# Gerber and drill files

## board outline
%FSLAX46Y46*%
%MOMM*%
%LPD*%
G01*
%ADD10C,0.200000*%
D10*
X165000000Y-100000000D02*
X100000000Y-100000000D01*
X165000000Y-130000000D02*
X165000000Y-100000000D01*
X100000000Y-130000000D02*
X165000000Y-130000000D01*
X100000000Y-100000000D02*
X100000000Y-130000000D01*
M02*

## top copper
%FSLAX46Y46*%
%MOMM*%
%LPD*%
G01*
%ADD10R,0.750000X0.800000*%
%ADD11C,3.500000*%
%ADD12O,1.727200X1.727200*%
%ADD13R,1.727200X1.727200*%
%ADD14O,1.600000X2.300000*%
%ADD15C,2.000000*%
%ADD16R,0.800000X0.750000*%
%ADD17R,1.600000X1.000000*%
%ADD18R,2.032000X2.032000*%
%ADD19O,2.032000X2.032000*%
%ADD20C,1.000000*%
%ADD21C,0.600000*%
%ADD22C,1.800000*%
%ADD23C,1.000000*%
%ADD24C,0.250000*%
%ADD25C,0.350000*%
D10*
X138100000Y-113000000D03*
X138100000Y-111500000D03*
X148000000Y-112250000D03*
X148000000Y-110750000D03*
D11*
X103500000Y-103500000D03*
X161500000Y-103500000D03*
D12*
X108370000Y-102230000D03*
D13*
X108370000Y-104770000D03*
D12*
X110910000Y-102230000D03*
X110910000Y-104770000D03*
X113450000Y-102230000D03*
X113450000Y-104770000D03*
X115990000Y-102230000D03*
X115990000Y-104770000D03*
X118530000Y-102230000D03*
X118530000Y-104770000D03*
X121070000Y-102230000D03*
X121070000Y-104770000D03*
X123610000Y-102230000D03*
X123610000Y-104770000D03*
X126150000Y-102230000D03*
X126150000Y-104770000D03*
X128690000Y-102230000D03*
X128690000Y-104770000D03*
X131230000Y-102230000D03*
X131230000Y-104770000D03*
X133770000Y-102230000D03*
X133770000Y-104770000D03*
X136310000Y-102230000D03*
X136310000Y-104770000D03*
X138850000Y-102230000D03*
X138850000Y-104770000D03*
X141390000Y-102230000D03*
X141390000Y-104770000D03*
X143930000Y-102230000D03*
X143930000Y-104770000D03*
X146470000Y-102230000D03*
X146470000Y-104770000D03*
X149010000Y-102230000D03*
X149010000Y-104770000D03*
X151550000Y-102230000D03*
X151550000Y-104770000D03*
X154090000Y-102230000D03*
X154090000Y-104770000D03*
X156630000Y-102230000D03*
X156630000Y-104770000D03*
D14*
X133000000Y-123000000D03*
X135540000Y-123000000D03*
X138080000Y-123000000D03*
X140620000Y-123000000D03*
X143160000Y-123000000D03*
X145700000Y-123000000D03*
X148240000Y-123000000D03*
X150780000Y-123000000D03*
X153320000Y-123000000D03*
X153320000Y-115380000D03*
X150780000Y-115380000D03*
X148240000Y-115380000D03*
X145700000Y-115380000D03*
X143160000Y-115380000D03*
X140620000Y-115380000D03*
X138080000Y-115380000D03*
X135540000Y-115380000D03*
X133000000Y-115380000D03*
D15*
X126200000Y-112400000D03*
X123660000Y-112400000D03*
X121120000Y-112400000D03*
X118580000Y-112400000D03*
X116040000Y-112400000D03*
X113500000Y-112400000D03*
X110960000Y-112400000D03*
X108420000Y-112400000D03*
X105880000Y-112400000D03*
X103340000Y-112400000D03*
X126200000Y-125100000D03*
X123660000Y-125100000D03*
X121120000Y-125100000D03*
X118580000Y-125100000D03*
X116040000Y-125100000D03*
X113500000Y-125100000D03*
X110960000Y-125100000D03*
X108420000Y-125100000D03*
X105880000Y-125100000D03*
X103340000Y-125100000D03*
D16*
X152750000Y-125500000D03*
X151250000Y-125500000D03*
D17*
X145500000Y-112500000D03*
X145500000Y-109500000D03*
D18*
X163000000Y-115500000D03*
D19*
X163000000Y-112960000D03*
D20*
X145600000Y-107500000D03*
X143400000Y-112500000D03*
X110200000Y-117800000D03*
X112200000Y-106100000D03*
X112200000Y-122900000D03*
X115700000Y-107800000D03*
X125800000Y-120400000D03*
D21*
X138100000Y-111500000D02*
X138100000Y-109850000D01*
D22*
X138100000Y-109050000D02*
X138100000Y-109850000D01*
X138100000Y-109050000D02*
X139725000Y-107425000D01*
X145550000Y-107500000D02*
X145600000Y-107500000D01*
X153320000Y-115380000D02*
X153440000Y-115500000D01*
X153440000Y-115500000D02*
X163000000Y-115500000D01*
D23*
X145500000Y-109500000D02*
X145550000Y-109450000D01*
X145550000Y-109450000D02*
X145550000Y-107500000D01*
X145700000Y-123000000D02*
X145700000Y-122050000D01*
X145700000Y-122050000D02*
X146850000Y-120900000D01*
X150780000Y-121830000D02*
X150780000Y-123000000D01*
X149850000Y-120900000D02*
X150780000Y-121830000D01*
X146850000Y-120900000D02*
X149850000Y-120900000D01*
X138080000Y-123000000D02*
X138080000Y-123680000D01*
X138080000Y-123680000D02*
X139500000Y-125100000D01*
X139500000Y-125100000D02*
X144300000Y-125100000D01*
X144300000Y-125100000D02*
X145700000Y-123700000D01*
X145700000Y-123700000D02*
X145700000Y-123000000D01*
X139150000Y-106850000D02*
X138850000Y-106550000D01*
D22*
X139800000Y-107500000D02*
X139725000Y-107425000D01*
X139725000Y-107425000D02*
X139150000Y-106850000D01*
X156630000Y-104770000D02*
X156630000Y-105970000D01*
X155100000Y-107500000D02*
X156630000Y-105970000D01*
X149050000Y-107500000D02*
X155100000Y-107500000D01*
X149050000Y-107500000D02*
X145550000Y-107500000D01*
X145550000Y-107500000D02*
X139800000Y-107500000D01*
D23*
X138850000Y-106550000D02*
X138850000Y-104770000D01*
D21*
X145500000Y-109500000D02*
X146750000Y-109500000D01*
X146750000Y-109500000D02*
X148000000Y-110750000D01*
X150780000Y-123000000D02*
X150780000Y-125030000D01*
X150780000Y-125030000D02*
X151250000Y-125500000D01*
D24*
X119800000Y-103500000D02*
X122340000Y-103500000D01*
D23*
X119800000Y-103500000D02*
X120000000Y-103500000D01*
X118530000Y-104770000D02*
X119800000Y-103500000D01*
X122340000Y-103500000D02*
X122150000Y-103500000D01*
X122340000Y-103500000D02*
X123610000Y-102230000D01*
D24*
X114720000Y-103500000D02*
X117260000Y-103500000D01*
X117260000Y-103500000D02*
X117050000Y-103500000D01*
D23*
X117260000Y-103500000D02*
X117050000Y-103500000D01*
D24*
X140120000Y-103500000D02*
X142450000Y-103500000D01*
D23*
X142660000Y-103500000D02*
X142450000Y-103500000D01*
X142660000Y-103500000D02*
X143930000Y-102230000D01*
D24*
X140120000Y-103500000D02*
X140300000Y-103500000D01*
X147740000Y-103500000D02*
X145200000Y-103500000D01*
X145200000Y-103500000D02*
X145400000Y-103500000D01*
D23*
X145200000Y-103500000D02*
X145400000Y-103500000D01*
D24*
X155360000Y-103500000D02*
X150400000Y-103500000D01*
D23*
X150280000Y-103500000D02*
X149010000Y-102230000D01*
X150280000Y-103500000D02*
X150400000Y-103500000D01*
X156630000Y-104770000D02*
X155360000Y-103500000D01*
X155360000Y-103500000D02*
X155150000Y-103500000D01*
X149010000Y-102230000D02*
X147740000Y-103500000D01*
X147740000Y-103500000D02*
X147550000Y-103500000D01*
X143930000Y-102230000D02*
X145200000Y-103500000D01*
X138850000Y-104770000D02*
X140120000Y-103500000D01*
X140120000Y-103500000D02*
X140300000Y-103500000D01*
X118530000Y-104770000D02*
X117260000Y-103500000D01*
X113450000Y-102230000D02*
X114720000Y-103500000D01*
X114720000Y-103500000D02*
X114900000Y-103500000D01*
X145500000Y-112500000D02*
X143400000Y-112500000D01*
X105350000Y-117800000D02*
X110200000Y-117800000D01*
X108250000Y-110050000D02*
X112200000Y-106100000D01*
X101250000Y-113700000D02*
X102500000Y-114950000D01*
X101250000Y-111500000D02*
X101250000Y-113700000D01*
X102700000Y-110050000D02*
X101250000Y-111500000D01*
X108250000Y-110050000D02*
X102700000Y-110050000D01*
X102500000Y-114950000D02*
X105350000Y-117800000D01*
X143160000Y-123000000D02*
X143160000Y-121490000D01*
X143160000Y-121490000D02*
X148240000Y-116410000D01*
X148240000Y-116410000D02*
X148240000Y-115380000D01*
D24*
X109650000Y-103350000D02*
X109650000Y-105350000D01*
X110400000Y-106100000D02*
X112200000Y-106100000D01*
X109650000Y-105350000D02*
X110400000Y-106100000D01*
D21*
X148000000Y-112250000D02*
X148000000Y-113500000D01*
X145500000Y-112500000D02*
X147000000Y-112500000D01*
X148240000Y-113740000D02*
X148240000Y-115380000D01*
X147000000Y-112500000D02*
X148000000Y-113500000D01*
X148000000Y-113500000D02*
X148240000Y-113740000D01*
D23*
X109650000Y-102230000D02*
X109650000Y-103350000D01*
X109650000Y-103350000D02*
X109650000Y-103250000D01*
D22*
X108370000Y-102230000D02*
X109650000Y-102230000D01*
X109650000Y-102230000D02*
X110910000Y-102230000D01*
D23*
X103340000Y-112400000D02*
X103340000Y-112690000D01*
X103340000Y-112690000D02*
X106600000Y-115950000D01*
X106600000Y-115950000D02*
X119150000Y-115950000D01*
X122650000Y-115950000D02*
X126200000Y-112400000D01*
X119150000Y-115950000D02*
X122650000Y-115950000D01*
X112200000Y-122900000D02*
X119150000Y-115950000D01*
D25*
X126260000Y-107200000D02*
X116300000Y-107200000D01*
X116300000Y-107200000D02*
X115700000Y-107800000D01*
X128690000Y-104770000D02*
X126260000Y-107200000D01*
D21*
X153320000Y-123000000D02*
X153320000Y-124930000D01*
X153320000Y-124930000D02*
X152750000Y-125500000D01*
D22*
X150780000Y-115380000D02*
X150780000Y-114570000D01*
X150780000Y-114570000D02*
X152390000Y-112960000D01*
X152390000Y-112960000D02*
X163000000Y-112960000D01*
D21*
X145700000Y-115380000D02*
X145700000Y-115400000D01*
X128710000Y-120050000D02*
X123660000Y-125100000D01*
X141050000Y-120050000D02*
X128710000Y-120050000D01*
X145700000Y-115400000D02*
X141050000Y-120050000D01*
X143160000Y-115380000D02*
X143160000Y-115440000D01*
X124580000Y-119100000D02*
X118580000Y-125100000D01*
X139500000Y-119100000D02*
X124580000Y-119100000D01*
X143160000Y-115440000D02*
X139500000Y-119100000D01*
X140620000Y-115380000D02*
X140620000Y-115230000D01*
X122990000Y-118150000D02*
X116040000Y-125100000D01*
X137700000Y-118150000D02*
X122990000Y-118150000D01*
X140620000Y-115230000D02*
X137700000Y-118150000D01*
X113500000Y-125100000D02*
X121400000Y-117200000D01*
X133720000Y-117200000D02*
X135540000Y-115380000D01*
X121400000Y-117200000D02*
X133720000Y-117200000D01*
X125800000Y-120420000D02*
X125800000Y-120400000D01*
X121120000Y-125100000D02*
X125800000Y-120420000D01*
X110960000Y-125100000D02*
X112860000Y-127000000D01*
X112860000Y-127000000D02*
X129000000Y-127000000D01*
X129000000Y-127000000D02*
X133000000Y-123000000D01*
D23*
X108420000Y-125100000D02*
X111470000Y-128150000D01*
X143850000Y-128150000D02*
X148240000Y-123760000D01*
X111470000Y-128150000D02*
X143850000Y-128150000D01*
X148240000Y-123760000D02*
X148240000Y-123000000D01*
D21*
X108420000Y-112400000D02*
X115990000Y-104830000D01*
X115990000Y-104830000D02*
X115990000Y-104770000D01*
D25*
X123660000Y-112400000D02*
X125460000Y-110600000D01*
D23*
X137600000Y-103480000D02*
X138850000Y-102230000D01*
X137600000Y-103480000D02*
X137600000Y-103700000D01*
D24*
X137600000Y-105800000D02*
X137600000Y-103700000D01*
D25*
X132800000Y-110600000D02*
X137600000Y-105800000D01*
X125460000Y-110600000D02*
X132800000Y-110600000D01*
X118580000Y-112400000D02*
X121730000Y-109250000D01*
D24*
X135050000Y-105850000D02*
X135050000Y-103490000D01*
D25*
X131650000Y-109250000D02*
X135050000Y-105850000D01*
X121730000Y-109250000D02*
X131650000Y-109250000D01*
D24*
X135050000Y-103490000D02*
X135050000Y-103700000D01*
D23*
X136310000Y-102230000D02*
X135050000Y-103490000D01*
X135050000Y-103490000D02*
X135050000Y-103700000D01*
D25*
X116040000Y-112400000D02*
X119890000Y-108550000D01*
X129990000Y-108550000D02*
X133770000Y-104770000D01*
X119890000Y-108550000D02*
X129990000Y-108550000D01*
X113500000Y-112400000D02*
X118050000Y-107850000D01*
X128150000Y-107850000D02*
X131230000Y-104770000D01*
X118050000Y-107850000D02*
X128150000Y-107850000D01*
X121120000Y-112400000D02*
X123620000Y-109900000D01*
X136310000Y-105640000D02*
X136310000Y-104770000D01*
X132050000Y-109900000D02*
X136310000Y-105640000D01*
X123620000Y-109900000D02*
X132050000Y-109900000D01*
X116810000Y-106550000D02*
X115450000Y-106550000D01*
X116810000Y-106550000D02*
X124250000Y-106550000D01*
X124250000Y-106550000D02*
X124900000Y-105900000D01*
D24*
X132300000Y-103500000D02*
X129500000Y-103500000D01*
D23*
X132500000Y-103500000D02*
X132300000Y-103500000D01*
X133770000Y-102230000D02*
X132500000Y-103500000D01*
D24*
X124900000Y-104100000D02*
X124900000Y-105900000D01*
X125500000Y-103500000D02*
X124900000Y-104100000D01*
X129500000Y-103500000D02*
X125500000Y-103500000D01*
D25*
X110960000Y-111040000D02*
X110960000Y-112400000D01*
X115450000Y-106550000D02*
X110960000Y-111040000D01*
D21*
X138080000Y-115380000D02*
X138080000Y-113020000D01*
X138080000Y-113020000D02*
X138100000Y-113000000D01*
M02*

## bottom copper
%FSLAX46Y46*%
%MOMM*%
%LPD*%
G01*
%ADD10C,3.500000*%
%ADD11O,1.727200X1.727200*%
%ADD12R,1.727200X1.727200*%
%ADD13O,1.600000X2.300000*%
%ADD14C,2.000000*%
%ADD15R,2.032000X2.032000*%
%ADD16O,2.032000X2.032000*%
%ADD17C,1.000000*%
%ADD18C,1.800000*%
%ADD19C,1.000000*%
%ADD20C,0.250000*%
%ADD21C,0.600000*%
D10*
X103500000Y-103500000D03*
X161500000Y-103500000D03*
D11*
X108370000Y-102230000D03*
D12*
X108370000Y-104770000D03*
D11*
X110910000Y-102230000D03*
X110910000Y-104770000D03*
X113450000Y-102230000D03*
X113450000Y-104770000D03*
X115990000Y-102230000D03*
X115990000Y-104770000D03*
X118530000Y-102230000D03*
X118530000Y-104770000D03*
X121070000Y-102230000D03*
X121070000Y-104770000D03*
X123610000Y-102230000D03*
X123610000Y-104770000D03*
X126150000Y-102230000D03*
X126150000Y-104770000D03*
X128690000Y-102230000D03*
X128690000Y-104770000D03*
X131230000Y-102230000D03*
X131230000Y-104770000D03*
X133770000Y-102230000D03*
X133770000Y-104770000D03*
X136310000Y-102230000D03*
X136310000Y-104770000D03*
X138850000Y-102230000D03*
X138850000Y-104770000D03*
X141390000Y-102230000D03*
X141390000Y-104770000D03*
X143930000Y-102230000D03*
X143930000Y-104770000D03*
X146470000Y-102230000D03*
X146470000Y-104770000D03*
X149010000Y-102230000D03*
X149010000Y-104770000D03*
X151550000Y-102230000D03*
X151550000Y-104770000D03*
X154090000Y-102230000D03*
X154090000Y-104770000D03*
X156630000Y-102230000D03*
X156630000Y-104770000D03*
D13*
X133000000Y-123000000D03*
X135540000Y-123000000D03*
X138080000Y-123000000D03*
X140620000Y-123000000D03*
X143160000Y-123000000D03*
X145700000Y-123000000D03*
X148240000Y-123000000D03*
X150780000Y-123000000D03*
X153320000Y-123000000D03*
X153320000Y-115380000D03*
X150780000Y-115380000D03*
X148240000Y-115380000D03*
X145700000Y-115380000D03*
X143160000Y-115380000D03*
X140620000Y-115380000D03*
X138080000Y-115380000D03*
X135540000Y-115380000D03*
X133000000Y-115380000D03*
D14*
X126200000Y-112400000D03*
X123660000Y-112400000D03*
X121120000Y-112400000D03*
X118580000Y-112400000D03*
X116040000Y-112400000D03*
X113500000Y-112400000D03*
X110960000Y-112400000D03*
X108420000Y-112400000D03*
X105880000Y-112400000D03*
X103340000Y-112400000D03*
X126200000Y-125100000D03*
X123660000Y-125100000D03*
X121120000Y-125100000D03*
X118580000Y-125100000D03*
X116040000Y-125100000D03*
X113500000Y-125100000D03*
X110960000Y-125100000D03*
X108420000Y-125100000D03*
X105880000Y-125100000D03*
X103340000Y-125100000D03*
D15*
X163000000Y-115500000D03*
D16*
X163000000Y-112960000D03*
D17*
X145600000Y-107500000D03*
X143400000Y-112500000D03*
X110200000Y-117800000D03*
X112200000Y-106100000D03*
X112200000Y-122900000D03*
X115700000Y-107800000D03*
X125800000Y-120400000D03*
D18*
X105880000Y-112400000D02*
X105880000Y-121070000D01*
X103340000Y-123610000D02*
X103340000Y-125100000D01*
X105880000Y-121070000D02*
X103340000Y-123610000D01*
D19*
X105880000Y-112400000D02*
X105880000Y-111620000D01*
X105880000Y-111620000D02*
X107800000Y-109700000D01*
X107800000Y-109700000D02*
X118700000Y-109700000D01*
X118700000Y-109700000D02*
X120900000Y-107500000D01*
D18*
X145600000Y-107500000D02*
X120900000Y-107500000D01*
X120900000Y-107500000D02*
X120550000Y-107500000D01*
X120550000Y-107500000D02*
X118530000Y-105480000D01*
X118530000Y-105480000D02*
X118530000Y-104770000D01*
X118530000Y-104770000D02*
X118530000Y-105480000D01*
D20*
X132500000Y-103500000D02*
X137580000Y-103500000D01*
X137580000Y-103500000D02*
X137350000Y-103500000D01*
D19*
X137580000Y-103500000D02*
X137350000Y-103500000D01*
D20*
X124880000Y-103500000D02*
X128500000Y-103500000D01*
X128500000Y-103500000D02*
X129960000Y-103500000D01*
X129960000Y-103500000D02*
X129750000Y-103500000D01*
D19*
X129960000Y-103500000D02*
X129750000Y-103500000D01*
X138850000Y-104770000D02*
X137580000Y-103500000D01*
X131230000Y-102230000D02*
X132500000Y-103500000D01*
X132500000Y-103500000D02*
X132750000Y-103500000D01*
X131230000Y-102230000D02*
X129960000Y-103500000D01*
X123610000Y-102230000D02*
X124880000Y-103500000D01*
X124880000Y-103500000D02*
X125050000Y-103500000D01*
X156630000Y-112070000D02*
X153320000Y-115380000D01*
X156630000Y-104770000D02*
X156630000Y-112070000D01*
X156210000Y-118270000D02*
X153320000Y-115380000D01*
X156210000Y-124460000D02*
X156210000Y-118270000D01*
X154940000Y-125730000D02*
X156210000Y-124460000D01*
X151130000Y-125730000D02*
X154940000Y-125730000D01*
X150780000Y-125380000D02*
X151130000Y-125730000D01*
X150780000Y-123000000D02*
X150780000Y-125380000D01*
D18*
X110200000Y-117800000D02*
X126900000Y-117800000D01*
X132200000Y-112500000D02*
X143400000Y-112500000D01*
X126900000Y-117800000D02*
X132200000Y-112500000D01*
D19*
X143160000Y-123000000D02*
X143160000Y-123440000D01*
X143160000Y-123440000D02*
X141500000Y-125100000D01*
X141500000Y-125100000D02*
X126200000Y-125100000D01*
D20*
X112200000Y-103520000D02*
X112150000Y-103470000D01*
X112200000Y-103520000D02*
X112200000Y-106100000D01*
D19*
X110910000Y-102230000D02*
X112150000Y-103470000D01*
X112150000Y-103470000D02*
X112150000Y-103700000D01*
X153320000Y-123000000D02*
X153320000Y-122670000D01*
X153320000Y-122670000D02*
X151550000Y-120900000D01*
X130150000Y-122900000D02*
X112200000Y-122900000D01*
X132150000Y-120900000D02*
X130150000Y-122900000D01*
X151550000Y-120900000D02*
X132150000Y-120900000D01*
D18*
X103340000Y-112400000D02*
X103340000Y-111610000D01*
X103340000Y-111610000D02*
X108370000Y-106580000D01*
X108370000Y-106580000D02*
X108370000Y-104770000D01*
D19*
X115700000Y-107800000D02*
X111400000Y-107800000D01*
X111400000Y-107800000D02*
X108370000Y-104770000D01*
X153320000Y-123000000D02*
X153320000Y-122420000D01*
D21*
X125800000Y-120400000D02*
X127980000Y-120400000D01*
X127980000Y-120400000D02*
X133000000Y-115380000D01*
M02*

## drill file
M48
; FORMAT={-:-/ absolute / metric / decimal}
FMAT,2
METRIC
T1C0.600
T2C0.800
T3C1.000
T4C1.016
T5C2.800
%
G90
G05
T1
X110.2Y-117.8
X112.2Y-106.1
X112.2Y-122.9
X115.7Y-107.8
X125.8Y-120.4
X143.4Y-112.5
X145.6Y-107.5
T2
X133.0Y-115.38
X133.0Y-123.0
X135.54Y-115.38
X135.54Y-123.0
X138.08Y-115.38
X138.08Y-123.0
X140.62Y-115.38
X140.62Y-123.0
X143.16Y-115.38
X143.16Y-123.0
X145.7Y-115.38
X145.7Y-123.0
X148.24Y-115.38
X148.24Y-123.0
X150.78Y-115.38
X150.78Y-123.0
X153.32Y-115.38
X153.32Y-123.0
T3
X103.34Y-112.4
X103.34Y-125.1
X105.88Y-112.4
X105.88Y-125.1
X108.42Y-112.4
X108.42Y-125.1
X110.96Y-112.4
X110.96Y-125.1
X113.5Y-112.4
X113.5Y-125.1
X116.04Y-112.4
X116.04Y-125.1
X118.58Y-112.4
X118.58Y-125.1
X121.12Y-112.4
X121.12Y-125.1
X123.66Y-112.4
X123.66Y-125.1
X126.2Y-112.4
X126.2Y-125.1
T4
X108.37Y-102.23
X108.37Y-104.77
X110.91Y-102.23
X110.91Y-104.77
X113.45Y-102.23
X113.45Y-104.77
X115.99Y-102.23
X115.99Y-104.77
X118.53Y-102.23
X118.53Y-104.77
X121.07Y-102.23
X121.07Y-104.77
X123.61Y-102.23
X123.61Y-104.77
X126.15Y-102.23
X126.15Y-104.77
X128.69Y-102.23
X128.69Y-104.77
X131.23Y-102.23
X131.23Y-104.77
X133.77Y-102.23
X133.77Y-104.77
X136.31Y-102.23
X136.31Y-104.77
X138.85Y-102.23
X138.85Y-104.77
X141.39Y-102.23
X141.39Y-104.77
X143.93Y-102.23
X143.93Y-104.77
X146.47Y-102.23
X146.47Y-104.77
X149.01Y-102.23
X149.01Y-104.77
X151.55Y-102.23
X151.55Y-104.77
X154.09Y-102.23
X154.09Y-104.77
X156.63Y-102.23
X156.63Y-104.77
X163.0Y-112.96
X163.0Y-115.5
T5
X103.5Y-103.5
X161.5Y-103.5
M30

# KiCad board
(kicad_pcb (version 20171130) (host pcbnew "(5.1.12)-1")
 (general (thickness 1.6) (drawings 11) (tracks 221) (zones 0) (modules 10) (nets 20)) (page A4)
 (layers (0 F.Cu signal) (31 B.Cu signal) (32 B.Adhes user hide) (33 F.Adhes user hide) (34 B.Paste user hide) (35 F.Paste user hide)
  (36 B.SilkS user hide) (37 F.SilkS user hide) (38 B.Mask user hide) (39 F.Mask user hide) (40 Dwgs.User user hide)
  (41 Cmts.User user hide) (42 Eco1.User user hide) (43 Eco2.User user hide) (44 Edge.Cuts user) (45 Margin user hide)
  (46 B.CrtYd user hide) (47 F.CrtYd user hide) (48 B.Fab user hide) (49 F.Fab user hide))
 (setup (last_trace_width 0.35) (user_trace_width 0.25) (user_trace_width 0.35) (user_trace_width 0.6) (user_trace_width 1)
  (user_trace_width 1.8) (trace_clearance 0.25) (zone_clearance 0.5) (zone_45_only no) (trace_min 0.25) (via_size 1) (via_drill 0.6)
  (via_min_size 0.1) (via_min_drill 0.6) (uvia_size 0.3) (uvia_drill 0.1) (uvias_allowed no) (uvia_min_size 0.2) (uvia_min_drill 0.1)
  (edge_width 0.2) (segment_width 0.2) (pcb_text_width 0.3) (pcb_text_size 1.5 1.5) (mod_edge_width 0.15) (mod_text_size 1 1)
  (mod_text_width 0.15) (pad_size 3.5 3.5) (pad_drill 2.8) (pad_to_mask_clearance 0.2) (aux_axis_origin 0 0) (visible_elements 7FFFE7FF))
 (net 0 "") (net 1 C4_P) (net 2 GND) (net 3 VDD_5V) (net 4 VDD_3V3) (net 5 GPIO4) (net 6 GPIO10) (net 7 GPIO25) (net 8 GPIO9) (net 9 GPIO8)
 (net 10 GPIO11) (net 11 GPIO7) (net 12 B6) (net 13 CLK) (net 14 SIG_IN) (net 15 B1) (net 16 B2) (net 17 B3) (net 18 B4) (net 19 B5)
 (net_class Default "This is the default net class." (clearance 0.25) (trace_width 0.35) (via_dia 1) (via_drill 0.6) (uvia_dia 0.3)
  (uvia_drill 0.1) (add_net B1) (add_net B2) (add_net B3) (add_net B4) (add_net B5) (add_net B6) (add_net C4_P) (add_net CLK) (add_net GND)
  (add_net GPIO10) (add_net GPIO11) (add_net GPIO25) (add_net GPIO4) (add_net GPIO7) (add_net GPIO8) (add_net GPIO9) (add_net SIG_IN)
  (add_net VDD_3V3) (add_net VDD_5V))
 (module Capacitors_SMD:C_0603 (layer F.Cu) (at 138.1 112.25 90)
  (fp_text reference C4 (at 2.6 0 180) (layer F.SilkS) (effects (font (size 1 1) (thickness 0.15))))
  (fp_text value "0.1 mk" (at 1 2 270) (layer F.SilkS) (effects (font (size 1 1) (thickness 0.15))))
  (pad 1 smd rect (at -0.75 0 90) (size 0.8 0.75) (layers F.Cu F.Paste F.Mask) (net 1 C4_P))
  (pad 2 smd rect (at 0.75 0 90) (size 0.8 0.75) (layers F.Cu F.Paste F.Mask) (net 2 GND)))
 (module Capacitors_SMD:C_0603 (layer F.Cu) (at 148 111.5 90)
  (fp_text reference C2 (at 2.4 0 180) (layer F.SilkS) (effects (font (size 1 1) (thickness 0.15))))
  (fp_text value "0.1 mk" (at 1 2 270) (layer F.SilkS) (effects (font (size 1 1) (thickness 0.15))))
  (pad 1 smd rect (at -0.75 0 90) (size 0.8 0.75) (layers F.Cu F.Paste F.Mask) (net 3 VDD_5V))
  (pad 2 smd rect (at 0.75 0 90) (size 0.8 0.75) (layers F.Cu F.Paste F.Mask) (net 2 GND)))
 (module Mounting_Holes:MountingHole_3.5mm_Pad (layer F.Cu) (at 103.5 103.5)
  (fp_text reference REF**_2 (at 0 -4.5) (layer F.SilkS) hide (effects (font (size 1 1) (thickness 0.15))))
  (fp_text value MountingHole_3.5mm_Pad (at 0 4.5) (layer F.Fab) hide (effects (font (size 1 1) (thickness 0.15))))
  (pad "" np_thru_hole circle (at 0 0) (size 3.5 3.5) (drill 2.8) (layers *.Cu *.Mask)))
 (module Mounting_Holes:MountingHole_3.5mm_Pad (layer F.Cu) (at 161.5 103.5)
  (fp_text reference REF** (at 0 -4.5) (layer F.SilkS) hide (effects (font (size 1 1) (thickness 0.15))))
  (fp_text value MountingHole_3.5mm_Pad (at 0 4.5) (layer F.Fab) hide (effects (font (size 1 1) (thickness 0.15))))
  (pad "" np_thru_hole circle (at 0 0) (size 3.5 3.5) (drill 2.8) (layers *.Cu *.Mask)))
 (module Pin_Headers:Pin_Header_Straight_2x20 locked (layer B.Cu) (at 108.37 102.23 270)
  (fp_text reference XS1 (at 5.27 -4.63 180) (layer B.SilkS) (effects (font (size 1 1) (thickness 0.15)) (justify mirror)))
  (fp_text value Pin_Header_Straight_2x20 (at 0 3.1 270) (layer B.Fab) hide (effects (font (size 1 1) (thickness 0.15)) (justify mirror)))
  (pad 2 thru_hole oval (at 0 0 270) (size 1.7272 1.7272) (drill 1.016) (layers *.Cu *.Mask B.SilkS) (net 3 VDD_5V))
  (pad 1 thru_hole rect (at 2.54 0 270) (size 1.7272 1.7272) (drill 1.016) (layers *.Cu *.Mask B.SilkS) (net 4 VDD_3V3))
  (pad 4 thru_hole oval (at 0 -2.54 270) (size 1.7272 1.7272) (drill 1.016) (layers *.Cu *.Mask B.SilkS) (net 3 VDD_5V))
  (pad 3 thru_hole oval (at 2.54 -2.54 270) (size 1.7272 1.7272) (drill 1.016) (layers *.Cu *.Mask B.SilkS))
  (pad 6 thru_hole oval (at 0 -5.08 270) (size 1.7272 1.7272) (drill 1.016) (layers *.Cu *.Mask B.SilkS) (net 2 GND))
  (pad 5 thru_hole oval (at 2.54 -5.08 270) (size 1.7272 1.7272) (drill 1.016) (layers *.Cu *.Mask B.SilkS))
  (pad 8 thru_hole oval (at 0 -7.62 270) (size 1.7272 1.7272) (drill 1.016) (layers *.Cu *.Mask B.SilkS))
  (pad 7 thru_hole oval (at 2.54 -7.62 270) (size 1.7272 1.7272) (drill 1.016) (layers *.Cu *.Mask B.SilkS) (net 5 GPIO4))
  (pad 10 thru_hole oval (at 0 -10.16 270) (size 1.7272 1.7272) (drill 1.016) (layers *.Cu *.Mask B.SilkS))
  (pad 9 thru_hole oval (at 2.54 -10.16 270) (size 1.7272 1.7272) (drill 1.016) (layers *.Cu *.Mask B.SilkS) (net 2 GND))
  (pad 12 thru_hole oval (at 0 -12.7 270) (size 1.7272 1.7272) (drill 1.016) (layers *.Cu *.Mask B.SilkS))
  (pad 11 thru_hole oval (at 2.54 -12.7 270) (size 1.7272 1.7272) (drill 1.016) (layers *.Cu *.Mask B.SilkS))
  (pad 14 thru_hole oval (at 0 -15.24 270) (size 1.7272 1.7272) (drill 1.016) (layers *.Cu *.Mask B.SilkS) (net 2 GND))
  (pad 13 thru_hole oval (at 2.54 -15.24 270) (size 1.7272 1.7272) (drill 1.016) (layers *.Cu *.Mask B.SilkS))
  (pad 16 thru_hole oval (at 0 -17.78 270) (size 1.7272 1.7272) (drill 1.016) (layers *.Cu *.Mask B.SilkS))
  (pad 15 thru_hole oval (at 2.54 -17.78 270) (size 1.7272 1.7272) (drill 1.016) (layers *.Cu *.Mask B.SilkS))
  (pad 18 thru_hole oval (at 0 -20.32 270) (size 1.7272 1.7272) (drill 1.016) (layers *.Cu *.Mask B.SilkS))
  (pad 17 thru_hole oval (at 2.54 -20.32 270) (size 1.7272 1.7272) (drill 1.016) (layers *.Cu *.Mask B.SilkS) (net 4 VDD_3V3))
  (pad 20 thru_hole oval (at 0 -22.86 270) (size 1.7272 1.7272) (drill 1.016) (layers *.Cu *.Mask B.SilkS) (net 2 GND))
  (pad 19 thru_hole oval (at 2.54 -22.86 270) (size 1.7272 1.7272) (drill 1.016) (layers *.Cu *.Mask B.SilkS) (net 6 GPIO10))
  (pad 22 thru_hole oval (at 0 -25.4 270) (size 1.7272 1.7272) (drill 1.016) (layers *.Cu *.Mask B.SilkS) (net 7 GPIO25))
  (pad 21 thru_hole oval (at 2.54 -25.4 270) (size 1.7272 1.7272) (drill 1.016) (layers *.Cu *.Mask B.SilkS) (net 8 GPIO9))
  (pad 24 thru_hole oval (at 0 -27.94 270) (size 1.7272 1.7272) (drill 1.016) (layers *.Cu *.Mask B.SilkS) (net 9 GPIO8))
  (pad 23 thru_hole oval (at 2.54 -27.94 270) (size 1.7272 1.7272) (drill 1.016) (layers *.Cu *.Mask B.SilkS) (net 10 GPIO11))
  (pad 26 thru_hole oval (at 0 -30.48 270) (size 1.7272 1.7272) (drill 1.016) (layers *.Cu *.Mask B.SilkS) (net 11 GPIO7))
  (pad 25 thru_hole oval (at 2.54 -30.48 270) (size 1.7272 1.7272) (drill 1.016) (layers *.Cu *.Mask B.SilkS) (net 2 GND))
  (pad 28 thru_hole oval (at 0 -33.02 270) (size 1.7272 1.7272) (drill 1.016) (layers *.Cu *.Mask B.SilkS))
  (pad 27 thru_hole oval (at 2.54 -33.02 270) (size 1.7272 1.7272) (drill 1.016) (layers *.Cu *.Mask B.SilkS))
  (pad 30 thru_hole oval (at 0 -35.56 270) (size 1.7272 1.7272) (drill 1.016) (layers *.Cu *.Mask B.SilkS) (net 2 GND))
  (pad 29 thru_hole oval (at 2.54 -35.56 270) (size 1.7272 1.7272) (drill 1.016) (layers *.Cu *.Mask B.SilkS))
  (pad 32 thru_hole oval (at 0 -38.1 270) (size 1.7272 1.7272) (drill 1.016) (layers *.Cu *.Mask B.SilkS))
  (pad 31 thru_hole oval (at 2.54 -38.1 270) (size 1.7272 1.7272) (drill 1.016) (layers *.Cu *.Mask B.SilkS))
  (pad 34 thru_hole oval (at 0 -40.64 270) (size 1.7272 1.7272) (drill 1.016) (layers *.Cu *.Mask B.SilkS) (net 2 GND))
  (pad 33 thru_hole oval (at 2.54 -40.64 270) (size 1.7272 1.7272) (drill 1.016) (layers *.Cu *.Mask B.SilkS))
  (pad 36 thru_hole oval (at 0 -43.18 270) (size 1.7272 1.7272) (drill 1.016) (layers *.Cu *.Mask B.SilkS))
  (pad 35 thru_hole oval (at 2.54 -43.18 270) (size 1.7272 1.7272) (drill 1.016) (layers *.Cu *.Mask B.SilkS))
  (pad 38 thru_hole oval (at 0 -45.72 270) (size 1.7272 1.7272) (drill 1.016) (layers *.Cu *.Mask B.SilkS))
  (pad 37 thru_hole oval (at 2.54 -45.72 270) (size 1.7272 1.7272) (drill 1.016) (layers *.Cu *.Mask B.SilkS))
  (pad 40 thru_hole oval (at 0 -48.26 270) (size 1.7272 1.7272) (drill 1.016) (layers *.Cu *.Mask B.SilkS))
  (pad 39 thru_hole oval (at 2.54 -48.26 270) (size 1.7272 1.7272) (drill 1.016) (layers *.Cu *.Mask B.SilkS) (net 2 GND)))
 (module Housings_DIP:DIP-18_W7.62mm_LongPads (layer F.Cu) (at 133 123 90)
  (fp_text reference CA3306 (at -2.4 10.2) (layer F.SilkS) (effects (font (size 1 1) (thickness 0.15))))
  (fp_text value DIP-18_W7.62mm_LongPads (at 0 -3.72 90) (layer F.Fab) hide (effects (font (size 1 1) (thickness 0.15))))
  (pad 1 thru_hole oval (at 0 0 90) (size 2.3 1.6) (drill 0.8) (layers *.Cu *.Mask F.SilkS) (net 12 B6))
  (pad 2 thru_hole oval (at 0 2.54 90) (size 2.3 1.6) (drill 0.8) (layers *.Cu *.Mask F.SilkS))
  (pad 3 thru_hole oval (at 0 5.08 90) (size 2.3 1.6) (drill 0.8) (layers *.Cu *.Mask F.SilkS) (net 2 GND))
  (pad 4 thru_hole oval (at 0 7.62 90) (size 2.3 1.6) (drill 0.8) (layers *.Cu *.Mask F.SilkS))
  (pad 5 thru_hole oval (at 0 10.16 90) (size 2.3 1.6) (drill 0.8) (layers *.Cu *.Mask F.SilkS) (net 3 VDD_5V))
  (pad 6 thru_hole oval (at 0 12.7 90) (size 2.3 1.6) (drill 0.8) (layers *.Cu *.Mask F.SilkS) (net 2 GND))
  (pad 7 thru_hole oval (at 0 15.24 90) (size 2.3 1.6) (drill 0.8) (layers *.Cu *.Mask F.SilkS) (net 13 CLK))
  (pad 8 thru_hole oval (at 0 17.78 90) (size 2.3 1.6) (drill 0.8) (layers *.Cu *.Mask F.SilkS) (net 2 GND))
  (pad 9 thru_hole oval (at 0 20.32 90) (size 2.3 1.6) (drill 0.8) (layers *.Cu *.Mask F.SilkS) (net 4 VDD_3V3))
  (pad 10 thru_hole oval (at 7.62 20.32 90) (size 2.3 1.6) (drill 0.8) (layers *.Cu *.Mask F.SilkS) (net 2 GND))
  (pad 11 thru_hole oval (at 7.62 17.78 90) (size 2.3 1.6) (drill 0.8) (layers *.Cu *.Mask F.SilkS) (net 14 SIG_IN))
  (pad 12 thru_hole oval (at 7.62 15.24 90) (size 2.3 1.6) (drill 0.8) (layers *.Cu *.Mask F.SilkS) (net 3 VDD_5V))
  (pad 13 thru_hole oval (at 7.62 12.7 90) (size 2.3 1.6) (drill 0.8) (layers *.Cu *.Mask F.SilkS) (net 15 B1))
  (pad 14 thru_hole oval (at 7.62 10.16 90) (size 2.3 1.6) (drill 0.8) (layers *.Cu *.Mask F.SilkS) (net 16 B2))
  (pad 15 thru_hole oval (at 7.62 7.62 90) (size 2.3 1.6) (drill 0.8) (layers *.Cu *.Mask F.SilkS) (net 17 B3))
  (pad 16 thru_hole oval (at 7.62 5.08 90) (size 2.3 1.6) (drill 0.8) (layers *.Cu *.Mask F.SilkS) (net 1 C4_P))
  (pad 17 thru_hole oval (at 7.62 2.54 90) (size 2.3 1.6) (drill 0.8) (layers *.Cu *.Mask F.SilkS) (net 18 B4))
  (pad 18 thru_hole oval (at 7.62 0 90) (size 2.3 1.6) (drill 0.8) (layers *.Cu *.Mask F.SilkS) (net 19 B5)))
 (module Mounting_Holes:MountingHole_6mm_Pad (layer F.Cu) (at 129 111 270)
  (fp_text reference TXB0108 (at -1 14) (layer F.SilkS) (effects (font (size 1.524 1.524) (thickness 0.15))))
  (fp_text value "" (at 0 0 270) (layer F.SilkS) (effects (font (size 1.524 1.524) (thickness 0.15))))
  (pad 1 thru_hole circle (at 1.4 2.8 270) (size 2 2) (drill 1) (layers *.Cu *.Mask F.SilkS) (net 4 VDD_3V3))
  (pad 2 thru_hole circle (at 1.4 5.34 270) (size 2 2) (drill 1) (layers *.Cu *.Mask F.SilkS) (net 11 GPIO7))
  (pad 3 thru_hole circle (at 1.4 7.88 270) (size 2 2) (drill 1) (layers *.Cu *.Mask F.SilkS) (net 10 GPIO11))
  (pad 4 thru_hole circle (at 1.4 10.42 270) (size 2 2) (drill 1) (layers *.Cu *.Mask F.SilkS) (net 9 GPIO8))
  (pad 5 thru_hole circle (at 1.4 12.96 270) (size 2 2) (drill 1) (layers *.Cu *.Mask F.SilkS) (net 8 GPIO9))
  (pad 6 thru_hole circle (at 1.4 15.5 270) (size 2 2) (drill 1) (layers *.Cu *.Mask F.SilkS) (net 6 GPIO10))
  (pad 7 thru_hole circle (at 1.4 18.04 270) (size 2 2) (drill 1) (layers *.Cu *.Mask F.SilkS) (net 7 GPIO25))
  (pad 8 thru_hole circle (at 1.4 20.58 270) (size 2 2) (drill 1) (layers *.Cu *.Mask F.SilkS) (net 5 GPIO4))
  (pad 9 thru_hole circle (at 1.4 23.12 270) (size 2 2) (drill 1) (layers *.Cu *.Mask F.SilkS) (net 2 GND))
  (pad 10 thru_hole circle (at 1.4 25.66 270) (size 2 2) (drill 1) (layers *.Cu *.Mask F.SilkS) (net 4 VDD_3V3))
  (pad 20 thru_hole circle (at 14.1 2.8 270) (size 2 2) (drill 1) (layers *.Cu *.Mask F.SilkS) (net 3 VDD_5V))
  (pad 19 thru_hole circle (at 14.1 5.34 270) (size 2 2) (drill 1) (layers *.Cu *.Mask F.SilkS) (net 15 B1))
  (pad 18 thru_hole circle (at 14.1 7.88 270) (size 2 2) (drill 1) (layers *.Cu *.Mask F.SilkS) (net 19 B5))
  (pad 17 thru_hole circle (at 14.1 10.42 270) (size 2 2) (drill 1) (layers *.Cu *.Mask F.SilkS) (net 16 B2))
  (pad 16 thru_hole circle (at 14.1 12.96 270) (size 2 2) (drill 1) (layers *.Cu *.Mask F.SilkS) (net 17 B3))
  (pad 15 thru_hole circle (at 14.1 15.5 270) (size 2 2) (drill 1) (layers *.Cu *.Mask F.SilkS) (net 18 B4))
  (pad 14 thru_hole circle (at 14.1 18.04 270) (size 2 2) (drill 1) (layers *.Cu *.Mask F.SilkS) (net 12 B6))
  (pad 13 thru_hole circle (at 14.1 20.58 270) (size 2 2) (drill 1) (layers *.Cu *.Mask F.SilkS) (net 13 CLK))
  (pad 12 thru_hole circle (at 14.1 23.12 270) (size 2 2) (drill 1) (layers *.Cu *.Mask F.SilkS))
  (pad 11 thru_hole circle (at 14.1 25.66 270) (size 2 2) (drill 1) (layers *.Cu *.Mask F.SilkS) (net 2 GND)))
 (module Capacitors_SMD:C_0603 (layer F.Cu) (at 152 125.5 180)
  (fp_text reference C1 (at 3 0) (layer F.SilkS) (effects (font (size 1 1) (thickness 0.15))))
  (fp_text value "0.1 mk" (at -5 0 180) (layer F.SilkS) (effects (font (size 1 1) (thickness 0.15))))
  (pad 1 smd rect (at -0.75 0 180) (size 0.8 0.75) (layers F.Cu F.Paste F.Mask) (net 4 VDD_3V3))
  (pad 2 smd rect (at 0.75 0 180) (size 0.8 0.75) (layers F.Cu F.Paste F.Mask) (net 2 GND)))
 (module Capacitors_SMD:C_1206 (layer F.Cu) (at 145.5 111 90)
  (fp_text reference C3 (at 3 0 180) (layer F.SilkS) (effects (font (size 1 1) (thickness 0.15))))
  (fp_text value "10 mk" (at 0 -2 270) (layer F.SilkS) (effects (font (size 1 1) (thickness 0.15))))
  (pad 1 smd rect (at -1.5 0 90) (size 1 1.6) (layers F.Cu F.Paste F.Mask) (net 3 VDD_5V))
  (pad 2 smd rect (at 1.5 0 90) (size 1 1.6) (layers F.Cu F.Paste F.Mask) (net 2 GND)))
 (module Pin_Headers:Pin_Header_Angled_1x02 (layer B.Cu) (at 163 115.5)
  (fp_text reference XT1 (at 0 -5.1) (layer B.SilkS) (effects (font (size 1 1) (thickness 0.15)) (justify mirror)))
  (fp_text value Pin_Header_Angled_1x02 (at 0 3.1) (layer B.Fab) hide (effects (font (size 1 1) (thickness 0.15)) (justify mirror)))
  (pad 1 thru_hole rect (at 0 0) (size 2.032 2.032) (drill 1.016) (layers *.Cu *.Mask B.SilkS) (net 2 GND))
  (pad 2 thru_hole oval (at 0 -2.54) (size 2.032 2.032) (drill 1.016) (layers *.Cu *.Mask B.SilkS) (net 14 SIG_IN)))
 (gr_line (start 165 100) (end 100 100) (angle 90) (layer Edge.Cuts) (width 0.2))
 (gr_line (start 165 130) (end 165 100) (angle 90) (layer Edge.Cuts) (width 0.2))
 (gr_line (start 100 130) (end 165 130) (angle 90) (layer Edge.Cuts) (width 0.2))
 (gr_line (start 100 100) (end 100 130) (angle 90) (layer Edge.Cuts) (width 0.2))
 (segment (start 138.1 111.5) (end 138.1 109.85) (width 0.6) (layer F.Cu) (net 2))
 (segment (start 138.1 109.05) (end 138.1 109.85) (width 1.8) (layer F.Cu) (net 2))
 (segment (start 138.1 109.05) (end 139.725 107.425) (width 1.8) (layer F.Cu) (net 2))
 (segment (start 105.88 112.4) (end 105.88 121.07) (width 1.8) (layer B.Cu) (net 2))
 (segment (start 103.34 123.61) (end 103.34 125.1) (width 1.8) (layer B.Cu) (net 2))
 (segment (start 105.88 121.07) (end 103.34 123.61) (width 1.8) (layer B.Cu) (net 2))
 (segment (start 105.88 112.4) (end 105.88 111.62) (width 1) (layer B.Cu) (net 2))
 (segment (start 105.88 111.62) (end 107.8 109.7) (width 1) (layer B.Cu) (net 2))
 (segment (start 107.8 109.7) (end 118.7 109.7) (width 1) (layer B.Cu) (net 2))
 (segment (start 118.7 109.7) (end 120.9 107.5) (width 1) (layer B.Cu) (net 2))
 (segment (start 145.6 107.5) (end 120.9 107.5) (width 1.8) (layer B.Cu) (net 2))
 (segment (start 120.9 107.5) (end 120.55 107.5) (width 1.8) (layer B.Cu) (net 2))
 (segment (start 145.55 107.5) (end 145.6 107.5) (width 1.8) (layer F.Cu) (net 2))
 (segment (start 120.55 107.5) (end 118.53 105.48) (width 1.8) (layer B.Cu) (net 2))
 (segment (start 118.53 105.48) (end 118.53 104.77) (width 1.8) (layer B.Cu) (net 2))
 (segment (start 118.53 104.77) (end 118.53 105.48) (width 1.8) (layer B.Cu) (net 2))
 (segment (start 153.32 115.38) (end 153.44 115.5) (width 1.8) (layer F.Cu) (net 2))
 (segment (start 153.44 115.5) (end 163 115.5) (width 1.8) (layer F.Cu) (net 2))
 (segment (start 145.5 109.5) (end 145.55 109.45) (width 1) (layer F.Cu) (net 2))
 (segment (start 145.55 109.45) (end 145.55 107.5) (width 1) (layer F.Cu) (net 2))
 (segment (start 145.7 123) (end 145.7 122.05) (width 1) (layer F.Cu) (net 2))
 (segment (start 145.7 122.05) (end 146.85 120.9) (width 1) (layer F.Cu) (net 2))
 (segment (start 150.78 121.83) (end 150.78 123) (width 1) (layer F.Cu) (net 2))
 (segment (start 149.85 120.9) (end 150.78 121.83) (width 1) (layer F.Cu) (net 2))
 (segment (start 146.85 120.9) (end 149.85 120.9) (width 1) (layer F.Cu) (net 2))
 (segment (start 138.08 123) (end 138.08 123.68) (width 1) (layer F.Cu) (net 2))
 (segment (start 138.08 123.68) (end 139.5 125.1) (width 1) (layer F.Cu) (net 2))
 (segment (start 139.5 125.1) (end 144.3 125.1) (width 1) (layer F.Cu) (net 2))
 (segment (start 144.3 125.1) (end 145.7 123.7) (width 1) (layer F.Cu) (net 2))
 (segment (start 145.7 123.7) (end 145.7 123) (width 1) (layer F.Cu) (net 2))
 (segment (start 139.15 106.85) (end 138.85 106.55) (width 1) (layer F.Cu) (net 2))
 (segment (start 139.8 107.5) (end 139.725 107.425) (width 1.8) (layer F.Cu) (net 2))
 (segment (start 139.725 107.425) (end 139.15 106.85) (width 1.8) (layer F.Cu) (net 2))
 (segment (start 156.63 104.77) (end 156.63 105.97) (width 1.8) (layer F.Cu) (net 2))
 (segment (start 155.1 107.5) (end 156.63 105.97) (width 1.8) (layer F.Cu) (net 2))
 (segment (start 149.05 107.5) (end 155.1 107.5) (width 1.8) (layer F.Cu) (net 2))
 (segment (start 149.05 107.5) (end 145.55 107.5) (width 1.8) (layer F.Cu) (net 2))
 (segment (start 145.55 107.5) (end 139.8 107.5) (width 1.8) (layer F.Cu) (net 2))
 (segment (start 138.85 106.55) (end 138.85 104.77) (width 1) (layer F.Cu) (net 2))
 (segment (start 145.5 109.5) (end 146.75 109.5) (width 0.6) (layer F.Cu) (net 2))
 (segment (start 146.75 109.5) (end 148 110.75) (width 0.6) (layer F.Cu) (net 2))
 (segment (start 150.78 123) (end 150.78 125.03) (width 0.6) (layer F.Cu) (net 2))
 (segment (start 150.78 125.03) (end 151.25 125.5) (width 0.6) (layer F.Cu) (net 2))
 (segment (start 132.5 103.5) (end 137.58 103.5) (width 0.25) (layer B.Cu) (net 2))
 (segment (start 137.58 103.5) (end 137.35 103.5) (width 0.25) (layer B.Cu) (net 2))
 (segment (start 137.58 103.5) (end 137.35 103.5) (width 1) (layer B.Cu) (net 2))
 (segment (start 124.88 103.5) (end 128.5 103.5) (width 0.25) (layer B.Cu) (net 2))
 (segment (start 128.5 103.5) (end 129.96 103.5) (width 0.25) (layer B.Cu) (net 2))
 (segment (start 129.96 103.5) (end 129.75 103.5) (width 0.25) (layer B.Cu) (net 2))
 (segment (start 129.96 103.5) (end 129.75 103.5) (width 1) (layer B.Cu) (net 2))
 (segment (start 119.8 103.5) (end 122.34 103.5) (width 0.25) (layer F.Cu) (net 2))
 (segment (start 119.8 103.5) (end 120 103.5) (width 1) (layer F.Cu) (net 2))
 (segment (start 118.53 104.77) (end 119.8 103.5) (width 1) (layer F.Cu) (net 2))
 (segment (start 122.34 103.5) (end 122.15 103.5) (width 1) (layer F.Cu) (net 2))
 (segment (start 122.34 103.5) (end 123.61 102.23) (width 1) (layer F.Cu) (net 2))
 (segment (start 114.72 103.5) (end 117.26 103.5) (width 0.25) (layer F.Cu) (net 2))
 (segment (start 117.26 103.5) (end 117.05 103.5) (width 0.25) (layer F.Cu) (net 2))
 (segment (start 117.26 103.5) (end 117.05 103.5) (width 1) (layer F.Cu) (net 2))
 (segment (start 140.12 103.5) (end 142.45 103.5) (width 0.25) (layer F.Cu) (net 2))
 (segment (start 142.66 103.5) (end 142.45 103.5) (width 1) (layer F.Cu) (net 2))
 (segment (start 142.66 103.5) (end 143.93 102.23) (width 1) (layer F.Cu) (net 2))
 (segment (start 140.12 103.5) (end 140.3 103.5) (width 0.25) (layer F.Cu) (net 2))
 (segment (start 147.74 103.5) (end 145.2 103.5) (width 0.25) (layer F.Cu) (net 2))
 (segment (start 145.2 103.5) (end 145.4 103.5) (width 0.25) (layer F.Cu) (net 2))
 (segment (start 145.2 103.5) (end 145.4 103.5) (width 1) (layer F.Cu) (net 2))
 (segment (start 155.36 103.5) (end 150.4 103.5) (width 0.25) (layer F.Cu) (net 2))
 (segment (start 150.28 103.5) (end 149.01 102.23) (width 1) (layer F.Cu) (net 2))
 (segment (start 150.28 103.5) (end 150.4 103.5) (width 1) (layer F.Cu) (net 2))
 (segment (start 156.63 104.77) (end 155.36 103.5) (width 1) (layer F.Cu) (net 2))
 (segment (start 155.36 103.5) (end 155.15 103.5) (width 1) (layer F.Cu) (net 2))
 (segment (start 149.01 102.23) (end 147.74 103.5) (width 1) (layer F.Cu) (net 2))
 (segment (start 147.74 103.5) (end 147.55 103.5) (width 1) (layer F.Cu) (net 2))
 (segment (start 143.93 102.23) (end 145.2 103.5) (width 1) (layer F.Cu) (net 2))
 (segment (start 138.85 104.77) (end 140.12 103.5) (width 1) (layer F.Cu) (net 2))
 (segment (start 140.12 103.5) (end 140.3 103.5) (width 1) (layer F.Cu) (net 2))
 (segment (start 138.85 104.77) (end 137.58 103.5) (width 1) (layer B.Cu) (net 2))
 (segment (start 131.23 102.23) (end 132.5 103.5) (width 1) (layer B.Cu) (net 2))
 (segment (start 132.5 103.5) (end 132.75 103.5) (width 1) (layer B.Cu) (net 2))
 (segment (start 131.23 102.23) (end 129.96 103.5) (width 1) (layer B.Cu) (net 2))
 (segment (start 123.61 102.23) (end 124.88 103.5) (width 1) (layer B.Cu) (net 2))
 (segment (start 124.88 103.5) (end 125.05 103.5) (width 1) (layer B.Cu) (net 2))
 (segment (start 118.53 104.77) (end 117.26 103.5) (width 1) (layer F.Cu) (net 2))
 (segment (start 113.45 102.23) (end 114.72 103.5) (width 1) (layer F.Cu) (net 2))
 (segment (start 114.72 103.5) (end 114.9 103.5) (width 1) (layer F.Cu) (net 2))
 (segment (start 156.63 112.07) (end 153.32 115.38) (width 1) (layer B.Cu) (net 2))
 (segment (start 156.63 104.77) (end 156.63 112.07) (width 1) (layer B.Cu) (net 2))
 (segment (start 156.21 118.27) (end 153.32 115.38) (width 1) (layer B.Cu) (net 2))
 (segment (start 156.21 124.46) (end 156.21 118.27) (width 1) (layer B.Cu) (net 2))
 (segment (start 154.94 125.73) (end 156.21 124.46) (width 1) (layer B.Cu) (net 2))
 (segment (start 151.13 125.73) (end 154.94 125.73) (width 1) (layer B.Cu) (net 2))
 (segment (start 150.78 125.38) (end 151.13 125.73) (width 1) (layer B.Cu) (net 2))
 (segment (start 150.78 123) (end 150.78 125.38) (width 1) (layer B.Cu) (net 2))
 (segment (start 110.2 117.8) (end 126.9 117.8) (width 1.8) (layer B.Cu) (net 3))
 (segment (start 145.5 112.5) (end 143.4 112.5) (width 1) (layer F.Cu) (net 3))
 (segment (start 105.35 117.8) (end 110.2 117.8) (width 1) (layer F.Cu) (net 3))
 (segment (start 108.25 110.05) (end 112.2 106.1) (width 1) (layer F.Cu) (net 3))
 (segment (start 101.25 113.7) (end 102.5 114.95) (width 1) (layer F.Cu) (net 3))
 (segment (start 101.25 111.5) (end 101.25 113.7) (width 1) (layer F.Cu) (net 3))
 (segment (start 102.7 110.05) (end 101.25 111.5) (width 1) (layer F.Cu) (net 3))
 (segment (start 108.25 110.05) (end 102.7 110.05) (width 1) (layer F.Cu) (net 3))
 (segment (start 102.5 114.95) (end 105.35 117.8) (width 1) (layer F.Cu) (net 3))
 (segment (start 132.2 112.5) (end 143.4 112.5) (width 1.8) (layer B.Cu) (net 3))
 (segment (start 126.9 117.8) (end 132.2 112.5) (width 1.8) (layer B.Cu) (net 3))
 (segment (start 143.16 123) (end 143.16 123.44) (width 1) (layer B.Cu) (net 3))
 (segment (start 143.16 123.44) (end 141.5 125.1) (width 1) (layer B.Cu) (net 3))
 (segment (start 141.5 125.1) (end 126.2 125.1) (width 1) (layer B.Cu) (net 3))
 (segment (start 143.16 123) (end 143.16 121.49) (width 1) (layer F.Cu) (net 3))
 (segment (start 143.16 121.49) (end 148.24 116.41) (width 1) (layer F.Cu) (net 3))
 (segment (start 148.24 116.41) (end 148.24 115.38) (width 1) (layer F.Cu) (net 3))
 (segment (start 109.65 103.35) (end 109.65 105.35) (width 0.25) (layer F.Cu) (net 3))
 (segment (start 110.4 106.1) (end 112.2 106.1) (width 0.25) (layer F.Cu) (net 3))
 (segment (start 109.65 105.35) (end 110.4 106.1) (width 0.25) (layer F.Cu) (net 3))
 (segment (start 112.2 103.52) (end 112.15 103.47) (width 0.25) (layer B.Cu) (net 3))
 (segment (start 112.2 103.52) (end 112.2 106.1) (width 0.25) (layer B.Cu) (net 3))
 (segment (start 148 112.25) (end 148 113.5) (width 0.6) (layer F.Cu) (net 3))
 (segment (start 145.5 112.5) (end 147 112.5) (width 0.6) (layer F.Cu) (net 3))
 (segment (start 148.24 113.74) (end 148.24 115.38) (width 0.6) (layer F.Cu) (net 3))
 (segment (start 147 112.5) (end 148 113.5) (width 0.6) (layer F.Cu) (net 3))
 (segment (start 148 113.5) (end 148.24 113.74) (width 0.6) (layer F.Cu) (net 3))
 (segment (start 110.91 102.23) (end 112.15 103.47) (width 1) (layer B.Cu) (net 3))
 (segment (start 112.15 103.47) (end 112.15 103.7) (width 1) (layer B.Cu) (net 3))
 (segment (start 109.65 102.23) (end 109.65 103.35) (width 1) (layer F.Cu) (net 3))
 (segment (start 109.65 103.35) (end 109.65 103.25) (width 1) (layer F.Cu) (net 3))
 (segment (start 108.37 102.23) (end 109.65 102.23) (width 1.8) (layer F.Cu) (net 3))
 (segment (start 109.65 102.23) (end 110.91 102.23) (width 1.8) (layer F.Cu) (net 3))
 (segment (start 103.34 112.4) (end 103.34 112.69) (width 1) (layer F.Cu) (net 4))
 (segment (start 103.34 112.69) (end 106.6 115.95) (width 1) (layer F.Cu) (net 4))
 (segment (start 106.6 115.95) (end 119.15 115.95) (width 1) (layer F.Cu) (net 4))
 (segment (start 153.32 123) (end 153.32 122.67) (width 1) (layer B.Cu) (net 4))
 (segment (start 153.32 122.67) (end 151.55 120.9) (width 1) (layer B.Cu) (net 4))
 (segment (start 122.65 115.95) (end 126.2 112.4) (width 1) (layer F.Cu) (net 4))
 (segment (start 119.15 115.95) (end 122.65 115.95) (width 1) (layer F.Cu) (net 4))
 (segment (start 112.2 122.9) (end 119.15 115.95) (width 1) (layer F.Cu) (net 4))
 (segment (start 130.15 122.9) (end 112.2 122.9) (width 1) (layer B.Cu) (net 4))
 (segment (start 132.15 120.9) (end 130.15 122.9) (width 1) (layer B.Cu) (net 4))
 (segment (start 151.55 120.9) (end 132.15 120.9) (width 1) (layer B.Cu) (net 4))
 (segment (start 103.34 112.4) (end 103.34 111.61) (width 1.8) (layer B.Cu) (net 4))
 (segment (start 103.34 111.61) (end 108.37 106.58) (width 1.8) (layer B.Cu) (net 4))
 (segment (start 108.37 106.58) (end 108.37 104.77) (width 1.8) (layer B.Cu) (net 4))
 (segment (start 115.7 107.8) (end 111.4 107.8) (width 1) (layer B.Cu) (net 4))
 (segment (start 126.26 107.2) (end 116.3 107.2) (width 0.35) (layer F.Cu) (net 4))
 (segment (start 116.3 107.2) (end 115.7 107.8) (width 0.35) (layer F.Cu) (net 4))
 (segment (start 128.69 104.77) (end 126.26 107.2) (width 0.35) (layer F.Cu) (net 4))
 (segment (start 111.4 107.8) (end 108.37 104.77) (width 1) (layer B.Cu) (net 4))
 (segment (start 153.32 123) (end 153.32 122.42) (width 1) (layer B.Cu) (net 4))
 (segment (start 153.32 123) (end 153.32 124.93) (width 0.6) (layer F.Cu) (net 4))
 (segment (start 153.32 124.93) (end 152.75 125.5) (width 0.6) (layer F.Cu) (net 4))
 (segment (start 150.78 115.38) (end 150.78 114.57) (width 1.8) (layer F.Cu) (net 14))
 (segment (start 150.78 114.57) (end 152.39 112.96) (width 1.8) (layer F.Cu) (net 14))
 (segment (start 152.39 112.96) (end 163 112.96) (width 1.8) (layer F.Cu) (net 14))
 (segment (start 145.7 115.38) (end 145.7 115.4) (width 0.6) (layer F.Cu) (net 15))
 (segment (start 128.71 120.05) (end 123.66 125.1) (width 0.6) (layer F.Cu) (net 15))
 (segment (start 141.05 120.05) (end 128.71 120.05) (width 0.6) (layer F.Cu) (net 15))
 (segment (start 145.7 115.4) (end 141.05 120.05) (width 0.6) (layer F.Cu) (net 15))
 (segment (start 143.16 115.38) (end 143.16 115.44) (width 0.6) (layer F.Cu) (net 16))
 (segment (start 124.58 119.1) (end 118.58 125.1) (width 0.6) (layer F.Cu) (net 16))
 (segment (start 139.5 119.1) (end 124.58 119.1) (width 0.6) (layer F.Cu) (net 16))
 (segment (start 143.16 115.44) (end 139.5 119.1) (width 0.6) (layer F.Cu) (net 16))
 (segment (start 140.62 115.38) (end 140.62 115.23) (width 0.6) (layer F.Cu) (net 17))
 (segment (start 122.99 118.15) (end 116.04 125.1) (width 0.6) (layer F.Cu) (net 17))
 (segment (start 137.7 118.15) (end 122.99 118.15) (width 0.6) (layer F.Cu) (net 17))
 (segment (start 140.62 115.23) (end 137.7 118.15) (width 0.6) (layer F.Cu) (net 17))
 (segment (start 113.5 125.1) (end 121.4 117.2) (width 0.6) (layer F.Cu) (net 18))
 (segment (start 133.72 117.2) (end 135.54 115.38) (width 0.6) (layer F.Cu) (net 18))
 (segment (start 121.4 117.2) (end 133.72 117.2) (width 0.6) (layer F.Cu) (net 18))
 (segment (start 125.8 120.4) (end 127.98 120.4) (width 0.6) (layer B.Cu) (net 19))
 (segment (start 125.8 120.42) (end 125.8 120.4) (width 0.6) (layer F.Cu) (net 19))
 (segment (start 121.12 125.1) (end 125.8 120.42) (width 0.6) (layer F.Cu) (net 19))
 (segment (start 127.98 120.4) (end 133 115.38) (width 0.6) (layer B.Cu) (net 19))
 (segment (start 110.96 125.1) (end 112.86 127) (width 0.6) (layer F.Cu) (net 12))
 (segment (start 112.86 127) (end 129 127) (width 0.6) (layer F.Cu) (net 12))
 (segment (start 129 127) (end 133 123) (width 0.6) (layer F.Cu) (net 12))
 (segment (start 108.42 125.1) (end 111.47 128.15) (width 1) (layer F.Cu) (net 13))
 (segment (start 143.85 128.15) (end 148.24 123.76) (width 1) (layer F.Cu) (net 13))
 (segment (start 111.47 128.15) (end 143.85 128.15) (width 1) (layer F.Cu) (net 13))
 (segment (start 148.24 123.76) (end 148.24 123) (width 1) (layer F.Cu) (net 13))
 (segment (start 108.42 112.4) (end 115.99 104.83) (width 0.6) (layer F.Cu) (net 5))
 (segment (start 115.99 104.83) (end 115.99 104.77) (width 0.6) (layer F.Cu) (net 5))
 (segment (start 123.66 112.4) (end 125.46 110.6) (width 0.35) (layer F.Cu) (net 11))
 (segment (start 137.6 103.48) (end 138.85 102.23) (width 1) (layer F.Cu) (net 11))
 (segment (start 137.6 103.48) (end 137.6 103.7) (width 1) (layer F.Cu) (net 11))
 (segment (start 137.6 105.8) (end 137.6 103.7) (width 0.25) (layer F.Cu) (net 11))
 (segment (start 132.8 110.6) (end 137.6 105.8) (width 0.35) (layer F.Cu) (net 11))
 (segment (start 125.46 110.6) (end 132.8 110.6) (width 0.35) (layer F.Cu) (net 11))
 (segment (start 118.58 112.4) (end 121.73 109.25) (width 0.35) (layer F.Cu) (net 9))
 (segment (start 135.05 105.85) (end 135.05 103.49) (width 0.25) (layer F.Cu) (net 9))
 (segment (start 131.65 109.25) (end 135.05 105.85) (width 0.35) (layer F.Cu) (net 9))
 (segment (start 121.73 109.25) (end 131.65 109.25) (width 0.35) (layer F.Cu) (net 9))
 (segment (start 135.05 103.49) (end 135.05 103.7) (width 0.25) (layer F.Cu) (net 9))
 (segment (start 136.31 102.23) (end 135.05 103.49) (width 1) (layer F.Cu) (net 9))
 (segment (start 135.05 103.49) (end 135.05 103.7) (width 1) (layer F.Cu) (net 9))
 (segment (start 116.04 112.4) (end 119.89 108.55) (width 0.35) (layer F.Cu) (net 8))
 (segment (start 129.99 108.55) (end 133.77 104.77) (width 0.35) (layer F.Cu) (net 8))
 (segment (start 119.89 108.55) (end 129.99 108.55) (width 0.35) (layer F.Cu) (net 8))
 (segment (start 113.5 112.4) (end 118.05 107.85) (width 0.35) (layer F.Cu) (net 6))
 (segment (start 128.15 107.85) (end 131.23 104.77) (width 0.35) (layer F.Cu) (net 6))
 (segment (start 118.05 107.85) (end 128.15 107.85) (width 0.35) (layer F.Cu) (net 6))
 (segment (start 121.12 112.4) (end 123.62 109.9) (width 0.35) (layer F.Cu) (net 10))
 (segment (start 136.31 105.64) (end 136.31 104.77) (width 0.35) (layer F.Cu) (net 10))
 (segment (start 132.05 109.9) (end 136.31 105.64) (width 0.35) (layer F.Cu) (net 10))
 (segment (start 123.62 109.9) (end 132.05 109.9) (width 0.35) (layer F.Cu) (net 10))
 (segment (start 116.81 106.55) (end 115.45 106.55) (width 0.35) (layer F.Cu) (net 7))
 (segment (start 116.81 106.55) (end 124.25 106.55) (width 0.35) (layer F.Cu) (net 7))
 (segment (start 124.25 106.55) (end 124.9 105.9) (width 0.35) (layer F.Cu) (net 7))
 (segment (start 132.3 103.5) (end 129.5 103.5) (width 0.25) (layer F.Cu) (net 7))
 (segment (start 132.5 103.5) (end 132.3 103.5) (width 1) (layer F.Cu) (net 7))
 (segment (start 133.77 102.23) (end 132.5 103.5) (width 1) (layer F.Cu) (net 7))
 (segment (start 124.9 104.1) (end 124.9 105.9) (width 0.25) (layer F.Cu) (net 7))
 (segment (start 125.5 103.5) (end 124.9 104.1) (width 0.25) (layer F.Cu) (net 7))
 (segment (start 129.5 103.5) (end 125.5 103.5) (width 0.25) (layer F.Cu) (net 7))
 (segment (start 110.96 111.04) (end 110.96 112.4) (width 0.35) (layer F.Cu) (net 7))
 (segment (start 115.45 106.55) (end 110.96 111.04) (width 0.35) (layer F.Cu) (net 7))
 (segment (start 138.08 115.38) (end 138.08 113.02) (width 0.6) (layer F.Cu) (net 1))
 (segment (start 138.08 113.02) (end 138.1 113) (width 0.6) (layer F.Cu) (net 1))
 (via (at 145.6 107.5) (size 1) (drill 0.6) (layers F.Cu B.Cu) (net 2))
 (via (at 143.4 112.5) (size 1) (drill 0.6) (layers F.Cu B.Cu) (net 3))
 (via (at 110.2 117.8) (size 1) (drill 0.6) (layers F.Cu B.Cu) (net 3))
 (via (at 112.2 106.1) (size 1) (drill 0.6) (layers F.Cu B.Cu) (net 3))
 (via (at 112.2 122.9) (size 1) (drill 0.6) (layers F.Cu B.Cu) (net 4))
 (via (at 115.7 107.8) (size 1) (drill 0.6) (layers F.Cu B.Cu) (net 4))
 (via (at 125.8 120.4) (size 1) (drill 0.6) (layers F.Cu B.Cu) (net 19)))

